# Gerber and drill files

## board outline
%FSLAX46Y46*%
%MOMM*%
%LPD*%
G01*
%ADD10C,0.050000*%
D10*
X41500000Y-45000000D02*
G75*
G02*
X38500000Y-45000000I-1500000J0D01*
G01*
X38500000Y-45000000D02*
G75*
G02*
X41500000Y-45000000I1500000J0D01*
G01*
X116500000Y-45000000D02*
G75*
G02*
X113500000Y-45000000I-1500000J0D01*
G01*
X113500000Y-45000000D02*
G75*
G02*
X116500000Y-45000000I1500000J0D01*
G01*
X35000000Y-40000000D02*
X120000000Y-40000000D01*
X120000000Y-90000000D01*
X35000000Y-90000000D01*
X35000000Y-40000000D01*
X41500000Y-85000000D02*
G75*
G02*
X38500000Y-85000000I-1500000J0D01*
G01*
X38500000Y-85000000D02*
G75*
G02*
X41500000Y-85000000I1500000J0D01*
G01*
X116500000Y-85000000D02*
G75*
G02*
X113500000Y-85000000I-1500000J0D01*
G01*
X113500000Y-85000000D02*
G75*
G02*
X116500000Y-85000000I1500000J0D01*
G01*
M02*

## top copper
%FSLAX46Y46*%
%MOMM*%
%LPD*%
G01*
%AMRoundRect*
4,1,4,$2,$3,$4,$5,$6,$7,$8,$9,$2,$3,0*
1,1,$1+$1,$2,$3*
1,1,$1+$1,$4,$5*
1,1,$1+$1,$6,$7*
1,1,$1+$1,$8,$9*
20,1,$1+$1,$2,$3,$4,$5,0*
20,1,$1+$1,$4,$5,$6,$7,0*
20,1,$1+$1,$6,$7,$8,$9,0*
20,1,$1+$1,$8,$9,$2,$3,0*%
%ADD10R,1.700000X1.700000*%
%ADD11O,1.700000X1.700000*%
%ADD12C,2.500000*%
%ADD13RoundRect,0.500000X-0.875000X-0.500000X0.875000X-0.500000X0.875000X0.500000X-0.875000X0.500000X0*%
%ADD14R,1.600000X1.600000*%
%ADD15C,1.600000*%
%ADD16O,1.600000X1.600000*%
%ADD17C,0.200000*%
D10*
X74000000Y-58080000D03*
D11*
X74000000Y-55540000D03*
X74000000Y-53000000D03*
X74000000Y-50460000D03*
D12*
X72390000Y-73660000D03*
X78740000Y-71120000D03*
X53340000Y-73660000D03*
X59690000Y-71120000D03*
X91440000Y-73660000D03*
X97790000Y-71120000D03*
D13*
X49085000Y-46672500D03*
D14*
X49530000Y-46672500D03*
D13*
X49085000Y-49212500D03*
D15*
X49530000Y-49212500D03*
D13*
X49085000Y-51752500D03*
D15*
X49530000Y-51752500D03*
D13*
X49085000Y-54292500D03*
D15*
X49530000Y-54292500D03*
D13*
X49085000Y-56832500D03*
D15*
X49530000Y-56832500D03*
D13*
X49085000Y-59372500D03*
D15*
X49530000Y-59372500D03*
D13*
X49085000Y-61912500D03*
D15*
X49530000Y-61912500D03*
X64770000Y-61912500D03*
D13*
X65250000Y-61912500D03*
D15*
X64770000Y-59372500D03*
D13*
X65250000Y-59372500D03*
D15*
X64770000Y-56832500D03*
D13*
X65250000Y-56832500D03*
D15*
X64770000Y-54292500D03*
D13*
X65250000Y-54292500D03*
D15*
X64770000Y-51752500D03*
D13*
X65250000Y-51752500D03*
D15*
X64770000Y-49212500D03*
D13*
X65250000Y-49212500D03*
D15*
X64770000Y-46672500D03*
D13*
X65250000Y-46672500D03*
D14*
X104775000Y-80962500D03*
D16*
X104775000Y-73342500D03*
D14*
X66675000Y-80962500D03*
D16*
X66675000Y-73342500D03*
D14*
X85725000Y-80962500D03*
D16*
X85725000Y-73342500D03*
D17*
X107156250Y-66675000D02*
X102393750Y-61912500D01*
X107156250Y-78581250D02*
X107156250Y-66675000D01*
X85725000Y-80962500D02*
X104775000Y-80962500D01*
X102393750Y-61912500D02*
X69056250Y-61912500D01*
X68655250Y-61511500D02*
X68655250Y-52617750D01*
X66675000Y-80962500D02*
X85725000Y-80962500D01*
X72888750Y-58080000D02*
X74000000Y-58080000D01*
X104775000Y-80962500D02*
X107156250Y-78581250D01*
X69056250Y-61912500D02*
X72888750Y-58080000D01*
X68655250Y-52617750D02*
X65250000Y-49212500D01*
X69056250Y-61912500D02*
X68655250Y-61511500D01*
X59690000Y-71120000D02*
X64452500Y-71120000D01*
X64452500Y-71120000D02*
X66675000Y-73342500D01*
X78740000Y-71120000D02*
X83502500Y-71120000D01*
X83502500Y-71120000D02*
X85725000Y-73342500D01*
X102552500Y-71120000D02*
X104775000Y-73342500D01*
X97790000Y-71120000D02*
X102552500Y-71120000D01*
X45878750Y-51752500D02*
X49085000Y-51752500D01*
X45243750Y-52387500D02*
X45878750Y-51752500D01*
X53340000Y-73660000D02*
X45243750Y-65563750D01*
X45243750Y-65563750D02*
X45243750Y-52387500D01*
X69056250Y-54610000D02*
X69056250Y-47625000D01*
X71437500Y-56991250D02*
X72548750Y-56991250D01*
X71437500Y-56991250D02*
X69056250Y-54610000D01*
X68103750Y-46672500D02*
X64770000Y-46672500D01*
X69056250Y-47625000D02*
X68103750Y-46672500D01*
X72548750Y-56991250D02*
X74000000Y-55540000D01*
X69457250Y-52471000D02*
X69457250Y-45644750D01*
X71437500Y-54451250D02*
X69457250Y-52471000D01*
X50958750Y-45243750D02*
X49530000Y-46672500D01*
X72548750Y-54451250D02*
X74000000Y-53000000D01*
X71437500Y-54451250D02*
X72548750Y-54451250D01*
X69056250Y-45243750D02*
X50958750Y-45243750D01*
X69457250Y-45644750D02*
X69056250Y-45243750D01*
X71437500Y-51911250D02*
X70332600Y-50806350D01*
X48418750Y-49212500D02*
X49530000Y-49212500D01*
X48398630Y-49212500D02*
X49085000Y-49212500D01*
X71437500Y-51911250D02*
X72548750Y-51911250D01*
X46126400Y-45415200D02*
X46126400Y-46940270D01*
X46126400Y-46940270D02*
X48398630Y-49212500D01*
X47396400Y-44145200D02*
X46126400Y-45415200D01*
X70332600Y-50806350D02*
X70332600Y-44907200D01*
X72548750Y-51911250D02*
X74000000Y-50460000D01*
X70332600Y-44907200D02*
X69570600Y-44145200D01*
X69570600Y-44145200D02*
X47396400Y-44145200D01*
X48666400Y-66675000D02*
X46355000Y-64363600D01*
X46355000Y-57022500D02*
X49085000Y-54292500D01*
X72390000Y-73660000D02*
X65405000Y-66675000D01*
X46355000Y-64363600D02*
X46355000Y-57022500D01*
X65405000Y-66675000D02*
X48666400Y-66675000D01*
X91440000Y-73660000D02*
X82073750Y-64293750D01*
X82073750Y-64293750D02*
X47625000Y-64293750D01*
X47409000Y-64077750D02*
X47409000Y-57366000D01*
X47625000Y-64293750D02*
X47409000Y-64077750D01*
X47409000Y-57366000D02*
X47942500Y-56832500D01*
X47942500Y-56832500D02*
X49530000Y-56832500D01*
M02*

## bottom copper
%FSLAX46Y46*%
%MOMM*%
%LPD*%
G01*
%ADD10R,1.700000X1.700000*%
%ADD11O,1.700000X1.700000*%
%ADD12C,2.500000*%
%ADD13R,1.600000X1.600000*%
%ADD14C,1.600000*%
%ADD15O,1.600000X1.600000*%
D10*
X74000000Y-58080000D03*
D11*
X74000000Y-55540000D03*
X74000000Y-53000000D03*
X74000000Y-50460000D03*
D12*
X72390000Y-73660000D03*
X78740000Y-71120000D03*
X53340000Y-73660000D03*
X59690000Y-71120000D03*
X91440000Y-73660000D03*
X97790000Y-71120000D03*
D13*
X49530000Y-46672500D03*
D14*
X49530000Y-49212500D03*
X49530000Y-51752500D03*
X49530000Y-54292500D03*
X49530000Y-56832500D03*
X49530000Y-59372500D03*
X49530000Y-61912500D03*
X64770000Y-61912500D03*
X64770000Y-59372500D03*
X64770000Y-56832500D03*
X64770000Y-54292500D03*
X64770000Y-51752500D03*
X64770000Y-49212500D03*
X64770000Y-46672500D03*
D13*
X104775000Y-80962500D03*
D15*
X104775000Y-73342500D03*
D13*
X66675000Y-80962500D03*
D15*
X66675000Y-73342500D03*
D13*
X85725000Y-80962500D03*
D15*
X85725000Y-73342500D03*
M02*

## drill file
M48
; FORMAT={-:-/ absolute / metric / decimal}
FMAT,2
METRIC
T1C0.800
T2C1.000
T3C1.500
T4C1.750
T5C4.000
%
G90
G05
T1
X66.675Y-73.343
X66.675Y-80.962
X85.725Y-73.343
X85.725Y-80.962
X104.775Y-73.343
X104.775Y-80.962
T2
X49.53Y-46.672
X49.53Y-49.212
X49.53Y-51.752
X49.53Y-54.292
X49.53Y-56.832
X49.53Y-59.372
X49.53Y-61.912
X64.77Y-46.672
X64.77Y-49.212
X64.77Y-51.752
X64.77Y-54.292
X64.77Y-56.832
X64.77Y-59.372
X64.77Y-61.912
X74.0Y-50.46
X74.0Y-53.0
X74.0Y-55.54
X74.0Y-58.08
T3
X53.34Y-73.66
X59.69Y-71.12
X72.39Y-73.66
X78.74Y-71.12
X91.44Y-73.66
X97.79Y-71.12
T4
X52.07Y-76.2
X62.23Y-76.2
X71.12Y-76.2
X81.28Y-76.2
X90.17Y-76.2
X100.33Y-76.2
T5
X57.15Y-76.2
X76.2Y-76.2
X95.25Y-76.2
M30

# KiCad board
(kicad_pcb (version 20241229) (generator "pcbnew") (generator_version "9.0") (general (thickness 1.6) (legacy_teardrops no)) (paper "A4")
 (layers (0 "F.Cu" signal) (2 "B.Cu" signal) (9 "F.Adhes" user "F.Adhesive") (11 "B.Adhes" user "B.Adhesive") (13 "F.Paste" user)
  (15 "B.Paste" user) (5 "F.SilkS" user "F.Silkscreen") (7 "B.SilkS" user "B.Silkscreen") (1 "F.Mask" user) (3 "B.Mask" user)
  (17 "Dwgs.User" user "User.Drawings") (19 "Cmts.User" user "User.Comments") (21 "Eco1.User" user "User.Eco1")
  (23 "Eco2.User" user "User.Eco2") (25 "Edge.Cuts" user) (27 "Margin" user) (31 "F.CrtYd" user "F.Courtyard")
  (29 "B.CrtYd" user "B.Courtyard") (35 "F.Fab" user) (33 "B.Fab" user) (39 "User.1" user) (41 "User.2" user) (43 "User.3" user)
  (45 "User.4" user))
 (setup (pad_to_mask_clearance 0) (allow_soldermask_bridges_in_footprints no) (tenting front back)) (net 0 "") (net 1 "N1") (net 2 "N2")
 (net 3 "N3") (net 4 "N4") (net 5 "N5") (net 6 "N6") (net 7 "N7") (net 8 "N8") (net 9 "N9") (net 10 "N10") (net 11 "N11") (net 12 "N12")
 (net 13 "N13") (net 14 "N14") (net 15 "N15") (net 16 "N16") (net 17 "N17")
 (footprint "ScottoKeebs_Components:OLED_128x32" (layer "F.Cu") (at 72.4 48.28)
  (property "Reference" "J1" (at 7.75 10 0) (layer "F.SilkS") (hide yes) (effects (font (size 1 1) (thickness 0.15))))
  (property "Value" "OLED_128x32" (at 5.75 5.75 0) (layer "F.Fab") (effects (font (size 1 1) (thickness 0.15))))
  (pad "1" thru_hole rect (at 1.6 9.8 180) (size 1.7 1.7) (drill 1) (layers "*.Cu" "*.Mask") (remove_unused_layers no) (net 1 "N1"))
  (pad "2" thru_hole oval (at 1.6 7.26 180) (size 1.7 1.7) (drill 1) (layers "*.Cu" "*.Mask") (remove_unused_layers no) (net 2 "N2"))
  (pad "3" thru_hole oval (at 1.6 4.72 180) (size 1.7 1.7) (drill 1) (layers "*.Cu" "*.Mask") (remove_unused_layers no) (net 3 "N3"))
  (pad "4" thru_hole oval (at 1.6 2.18 180) (size 1.7 1.7) (drill 1) (layers "*.Cu" "*.Mask") (remove_unused_layers no) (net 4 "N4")))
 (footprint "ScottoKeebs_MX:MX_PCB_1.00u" (layer "F.Cu") (at 76.2 76.2)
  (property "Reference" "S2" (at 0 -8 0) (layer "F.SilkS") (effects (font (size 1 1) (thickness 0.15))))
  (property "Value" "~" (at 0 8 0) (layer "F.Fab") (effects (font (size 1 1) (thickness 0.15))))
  (pad "" np_thru_hole circle (at -5.08 0) (size 1.75 1.75) (drill 1.75) (layers "*.Cu" "*.Mask"))
  (pad "" np_thru_hole circle (at 0 0) (size 4 4) (drill 4) (layers "*.Cu" "*.Mask"))
  (pad "" np_thru_hole circle (at 5.08 0) (size 1.75 1.75) (drill 1.75) (layers "*.Cu" "*.Mask"))
  (pad "1" thru_hole circle (at -3.81 -2.54) (size 2.5 2.5) (drill 1.5) (layers "*.Cu" "*.Mask") (remove_unused_layers no) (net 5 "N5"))
  (pad "2" thru_hole circle (at 2.54 -5.08) (size 2.5 2.5) (drill 1.5) (layers "*.Cu" "*.Mask") (remove_unused_layers no) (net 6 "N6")))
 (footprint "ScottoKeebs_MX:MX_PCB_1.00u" (layer "F.Cu") (at 57.15 76.2)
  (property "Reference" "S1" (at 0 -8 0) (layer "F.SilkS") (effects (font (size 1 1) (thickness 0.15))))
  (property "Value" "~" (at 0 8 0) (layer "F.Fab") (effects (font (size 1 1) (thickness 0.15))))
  (pad "" np_thru_hole circle (at -5.08 0) (size 1.75 1.75) (drill 1.75) (layers "*.Cu" "*.Mask"))
  (pad "" np_thru_hole circle (at 0 0) (size 4 4) (drill 4) (layers "*.Cu" "*.Mask"))
  (pad "" np_thru_hole circle (at 5.08 0) (size 1.75 1.75) (drill 1.75) (layers "*.Cu" "*.Mask"))
  (pad "1" thru_hole circle (at -3.81 -2.54) (size 2.5 2.5) (drill 1.5) (layers "*.Cu" "*.Mask") (remove_unused_layers no) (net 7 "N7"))
  (pad "2" thru_hole circle (at 2.54 -5.08) (size 2.5 2.5) (drill 1.5) (layers "*.Cu" "*.Mask") (remove_unused_layers no) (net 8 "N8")))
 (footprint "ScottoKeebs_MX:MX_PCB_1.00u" (layer "F.Cu") (at 95.25 76.2)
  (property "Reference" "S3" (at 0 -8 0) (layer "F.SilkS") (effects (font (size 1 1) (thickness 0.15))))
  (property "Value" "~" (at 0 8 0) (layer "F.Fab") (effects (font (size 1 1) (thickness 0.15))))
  (pad "" np_thru_hole circle (at -5.08 0) (size 1.75 1.75) (drill 1.75) (layers "*.Cu" "*.Mask"))
  (pad "" np_thru_hole circle (at 0 0) (size 4 4) (drill 4) (layers "*.Cu" "*.Mask"))
  (pad "" np_thru_hole circle (at 5.08 0) (size 1.75 1.75) (drill 1.75) (layers "*.Cu" "*.Mask"))
  (pad "1" thru_hole circle (at -3.81 -2.54) (size 2.5 2.5) (drill 1.5) (layers "*.Cu" "*.Mask") (remove_unused_layers no) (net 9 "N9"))
  (pad "2" thru_hole circle (at 2.54 -5.08) (size 2.5 2.5) (drill 1.5) (layers "*.Cu" "*.Mask") (remove_unused_layers no) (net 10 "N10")))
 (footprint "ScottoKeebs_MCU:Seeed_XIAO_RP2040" (layer "F.Cu") (at 57.15 54.2925)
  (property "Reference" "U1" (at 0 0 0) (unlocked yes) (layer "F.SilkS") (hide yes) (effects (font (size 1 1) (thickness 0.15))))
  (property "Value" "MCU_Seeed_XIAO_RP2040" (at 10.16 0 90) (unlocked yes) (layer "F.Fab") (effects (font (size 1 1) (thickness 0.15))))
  (pad "1" smd roundrect (at -8.065 -7.62) (size 2.75 2) (layers "F.Cu" "F.Mask" "F.Paste") (roundrect_rratio 0.25) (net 3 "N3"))
  (pad "1" thru_hole rect (at -7.62 -7.62 90) (size 1.6 1.6) (drill 1) (layers "*.Cu" "*.Mask") (remove_unused_layers no) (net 3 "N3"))
  (pad "2" smd roundrect (at -8.065 -5.08) (size 2.75 2) (layers "F.Cu" "F.Mask" "F.Paste") (roundrect_rratio 0.25) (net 4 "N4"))
  (pad "2" thru_hole circle (at -7.62 -5.08 90) (size 1.6 1.6) (drill 1) (layers "*.Cu" "*.Mask") (remove_unused_layers no) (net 4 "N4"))
  (pad "3" smd roundrect (at -8.065 -2.54) (size 2.75 2) (layers "F.Cu" "F.Mask" "F.Paste") (roundrect_rratio 0.25) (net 7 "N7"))
  (pad "3" thru_hole circle (at -7.62 -2.54 90) (size 1.6 1.6) (drill 1) (layers "*.Cu" "*.Mask") (remove_unused_layers no) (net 7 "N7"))
  (pad "4" smd roundrect (at -8.065 0) (size 2.75 2) (layers "F.Cu" "F.Mask" "F.Paste") (roundrect_rratio 0.25) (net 5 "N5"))
  (pad "4" thru_hole circle (at -7.62 0 90) (size 1.6 1.6) (drill 1) (layers "*.Cu" "*.Mask") (remove_unused_layers no) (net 5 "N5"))
  (pad "5" smd roundrect (at -8.065 2.54) (size 2.75 2) (layers "F.Cu" "F.Mask" "F.Paste") (roundrect_rratio 0.25) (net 9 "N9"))
  (pad "5" thru_hole circle (at -7.62 2.54 90) (size 1.6 1.6) (drill 1) (layers "*.Cu" "*.Mask") (remove_unused_layers no) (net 9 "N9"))
  (pad "6" smd roundrect (at -8.065 5.08) (size 2.75 2) (layers "F.Cu" "F.Mask" "F.Paste") (roundrect_rratio 0.25) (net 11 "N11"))
  (pad "6" thru_hole circle (at -7.62 5.08 90) (size 1.6 1.6) (drill 1) (layers "*.Cu" "*.Mask") (remove_unused_layers no) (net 11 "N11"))
  (pad "7" smd roundrect (at -8.065 7.62) (size 2.75 2) (layers "F.Cu" "F.Mask" "F.Paste") (roundrect_rratio 0.25) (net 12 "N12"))
  (pad "7" thru_hole circle (at -7.62 7.62 90) (size 1.6 1.6) (drill 1) (layers "*.Cu" "*.Mask") (remove_unused_layers no) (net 12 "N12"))
  (pad "8" thru_hole circle (at 7.62 7.62 90) (size 1.6 1.6) (drill 1) (layers "*.Cu" "*.Mask") (remove_unused_layers no) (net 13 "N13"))
  (pad "8" smd roundrect (at 8.1 7.62) (size 2.75 2) (layers "F.Cu" "F.Mask" "F.Paste") (roundrect_rratio 0.25) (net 13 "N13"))
  (pad "9" thru_hole circle (at 7.62 5.08 90) (size 1.6 1.6) (drill 1) (layers "*.Cu" "*.Mask") (remove_unused_layers no) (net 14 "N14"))
  (pad "9" smd roundrect (at 8.1 5.08) (size 2.75 2) (layers "F.Cu" "F.Mask" "F.Paste") (roundrect_rratio 0.25) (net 14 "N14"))
  (pad "10" thru_hole circle (at 7.62 2.54 90) (size 1.6 1.6) (drill 1) (layers "*.Cu" "*.Mask") (remove_unused_layers no) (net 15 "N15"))
  (pad "10" smd roundrect (at 8.1 2.54) (size 2.75 2) (layers "F.Cu" "F.Mask" "F.Paste") (roundrect_rratio 0.25) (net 15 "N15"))
  (pad "11" thru_hole circle (at 7.62 0 90) (size 1.6 1.6) (drill 1) (layers "*.Cu" "*.Mask") (remove_unused_layers no) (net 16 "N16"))
  (pad "11" smd roundrect (at 8.1 0) (size 2.75 2) (layers "F.Cu" "F.Mask" "F.Paste") (roundrect_rratio 0.25) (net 16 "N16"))
  (pad "12" thru_hole circle (at 7.62 -2.54 90) (size 1.6 1.6) (drill 1) (layers "*.Cu" "*.Mask") (remove_unused_layers no) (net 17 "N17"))
  (pad "12" smd roundrect (at 8.1 -2.54) (size 2.75 2) (layers "F.Cu" "F.Mask" "F.Paste") (roundrect_rratio 0.25) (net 17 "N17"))
  (pad "13" thru_hole circle (at 7.62 -5.08 90) (size 1.6 1.6) (drill 1) (layers "*.Cu" "*.Mask") (remove_unused_layers no) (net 1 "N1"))
  (pad "13" smd roundrect (at 8.1 -5.08) (size 2.75 2) (layers "F.Cu" "F.Mask" "F.Paste") (roundrect_rratio 0.25) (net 1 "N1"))
  (pad "14" thru_hole circle (at 7.62 -7.62 90) (size 1.6 1.6) (drill 1) (layers "*.Cu" "*.Mask") (remove_unused_layers no) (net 2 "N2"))
  (pad "14" smd roundrect (at 8.1 -7.62) (size 2.75 2) (layers "F.Cu" "F.Mask" "F.Paste") (roundrect_rratio 0.25) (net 2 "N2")))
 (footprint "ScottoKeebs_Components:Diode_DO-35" (layer "B.Cu") (at 104.775 80.9625 90)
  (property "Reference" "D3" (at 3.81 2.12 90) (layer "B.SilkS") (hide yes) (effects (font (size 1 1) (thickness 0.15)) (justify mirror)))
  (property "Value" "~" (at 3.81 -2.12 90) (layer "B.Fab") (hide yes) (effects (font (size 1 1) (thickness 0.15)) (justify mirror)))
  (pad "1" thru_hole rect (at 0 0 90) (size 1.6 1.6) (drill 0.8) (layers "*.Cu" "*.Mask") (remove_unused_layers no) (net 1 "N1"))
  (pad "2" thru_hole oval (at 7.62 0 90) (size 1.6 1.6) (drill 0.8) (layers "*.Cu" "*.Mask") (remove_unused_layers no) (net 10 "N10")))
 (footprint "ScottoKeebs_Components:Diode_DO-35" (layer "B.Cu") (at 66.675 80.9625 90)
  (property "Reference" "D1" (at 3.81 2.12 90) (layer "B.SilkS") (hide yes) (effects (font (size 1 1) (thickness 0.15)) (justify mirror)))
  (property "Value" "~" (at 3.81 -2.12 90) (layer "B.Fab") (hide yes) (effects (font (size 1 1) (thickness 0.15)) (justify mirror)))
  (pad "1" thru_hole rect (at 0 0 90) (size 1.6 1.6) (drill 0.8) (layers "*.Cu" "*.Mask") (remove_unused_layers no) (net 1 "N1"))
  (pad "2" thru_hole oval (at 7.62 0 90) (size 1.6 1.6) (drill 0.8) (layers "*.Cu" "*.Mask") (remove_unused_layers no) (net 8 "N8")))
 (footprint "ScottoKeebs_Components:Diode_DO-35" (layer "B.Cu") (at 85.725 80.9625 90)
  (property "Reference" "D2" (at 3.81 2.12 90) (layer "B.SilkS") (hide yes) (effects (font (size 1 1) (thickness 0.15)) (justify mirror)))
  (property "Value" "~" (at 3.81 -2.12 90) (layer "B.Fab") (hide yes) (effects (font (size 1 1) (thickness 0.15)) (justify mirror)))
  (pad "1" thru_hole rect (at 0 0 90) (size 1.6 1.6) (drill 0.8) (layers "*.Cu" "*.Mask") (remove_unused_layers no) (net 1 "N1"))
  (pad "2" thru_hole oval (at 7.62 0 90) (size 1.6 1.6) (drill 0.8) (layers "*.Cu" "*.Mask") (remove_unused_layers no) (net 6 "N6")))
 (gr_circle (center 40 45) (end 40 46.5) (stroke (width 0.05) (type default)) (fill no) (layer "Edge.Cuts"))
 (gr_circle (center 115 45) (end 115 46.5) (stroke (width 0.05) (type default)) (fill no) (layer "Edge.Cuts"))
 (gr_rect (start 35 40) (end 120 90) (stroke (width 0.05) (type default)) (fill no) (layer "Edge.Cuts"))
 (gr_circle (center 40 85) (end 40 86.5) (stroke (width 0.05) (type default)) (fill no) (layer "Edge.Cuts"))
 (gr_circle (center 115 85) (end 115 86.5) (stroke (width 0.05) (type default)) (fill no) (layer "Edge.Cuts"))
 (segment (start 107.15625 66.675) (end 102.39375 61.9125) (width 0.2) (layer "F.Cu") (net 1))
 (segment (start 107.15625 78.58125) (end 107.15625 66.675) (width 0.2) (layer "F.Cu") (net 1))
 (segment (start 85.725 80.9625) (end 104.775 80.9625) (width 0.2) (layer "F.Cu") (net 1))
 (segment (start 102.39375 61.9125) (end 69.05625 61.9125) (width 0.2) (layer "F.Cu") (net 1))
 (segment (start 68.65525 61.5115) (end 68.65525 52.61775) (width 0.2) (layer "F.Cu") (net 1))
 (segment (start 66.675 80.9625) (end 85.725 80.9625) (width 0.2) (layer "F.Cu") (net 1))
 (segment (start 72.88875 58.08) (end 74 58.08) (width 0.2) (layer "F.Cu") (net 1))
 (segment (start 104.775 80.9625) (end 107.15625 78.58125) (width 0.2) (layer "F.Cu") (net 1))
 (segment (start 69.05625 61.9125) (end 72.88875 58.08) (width 0.2) (layer "F.Cu") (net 1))
 (segment (start 68.65525 52.61775) (end 65.25 49.2125) (width 0.2) (layer "F.Cu") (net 1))
 (segment (start 69.05625 61.9125) (end 68.65525 61.5115) (width 0.2) (layer "F.Cu") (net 1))
 (segment (start 59.69 71.12) (end 64.4525 71.12) (width 0.2) (layer "F.Cu") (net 8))
 (segment (start 64.4525 71.12) (end 66.675 73.3425) (width 0.2) (layer "F.Cu") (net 8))
 (segment (start 78.74 71.12) (end 83.5025 71.12) (width 0.2) (layer "F.Cu") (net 6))
 (segment (start 83.5025 71.12) (end 85.725 73.3425) (width 0.2) (layer "F.Cu") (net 6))
 (segment (start 102.5525 71.12) (end 104.775 73.3425) (width 0.2) (layer "F.Cu") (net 10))
 (segment (start 97.79 71.12) (end 102.5525 71.12) (width 0.2) (layer "F.Cu") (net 10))
 (segment (start 45.87875 51.7525) (end 49.085 51.7525) (width 0.2) (layer "F.Cu") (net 7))
 (segment (start 45.24375 52.3875) (end 45.87875 51.7525) (width 0.2) (layer "F.Cu") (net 7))
 (segment (start 53.34 73.66) (end 45.24375 65.56375) (width 0.2) (layer "F.Cu") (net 7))
 (segment (start 45.24375 65.56375) (end 45.24375 52.3875) (width 0.2) (layer "F.Cu") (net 7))
 (segment (start 69.05625 54.61) (end 69.05625 47.625) (width 0.2) (layer "F.Cu") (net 2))
 (segment (start 71.4375 56.99125) (end 72.54875 56.99125) (width 0.2) (layer "F.Cu") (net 2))
 (segment (start 71.4375 56.99125) (end 69.05625 54.61) (width 0.2) (layer "F.Cu") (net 2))
 (segment (start 68.10375 46.6725) (end 64.77 46.6725) (width 0.2) (layer "F.Cu") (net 2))
 (segment (start 69.05625 47.625) (end 68.10375 46.6725) (width 0.2) (layer "F.Cu") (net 2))
 (segment (start 72.54875 56.99125) (end 74 55.54) (width 0.2) (layer "F.Cu") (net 2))
 (segment (start 69.45725 52.471) (end 69.45725 45.64475) (width 0.2) (layer "F.Cu") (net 3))
 (segment (start 71.4375 54.45125) (end 69.45725 52.471) (width 0.2) (layer "F.Cu") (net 3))
 (segment (start 50.95875 45.24375) (end 49.53 46.6725) (width 0.2) (layer "F.Cu") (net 3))
 (segment (start 72.54875 54.45125) (end 74 53) (width 0.2) (layer "F.Cu") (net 3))
 (segment (start 71.4375 54.45125) (end 72.54875 54.45125) (width 0.2) (layer "F.Cu") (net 3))
 (segment (start 69.05625 45.24375) (end 50.95875 45.24375) (width 0.2) (layer "F.Cu") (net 3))
 (segment (start 69.45725 45.64475) (end 69.05625 45.24375) (width 0.2) (layer "F.Cu") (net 3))
 (segment (start 71.4375 51.91125) (end 70.3326 50.80635) (width 0.2) (layer "F.Cu") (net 4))
 (segment (start 48.41875 49.2125) (end 49.53 49.2125) (width 0.2) (layer "F.Cu") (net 4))
 (segment (start 48.39863 49.2125) (end 49.085 49.2125) (width 0.2) (layer "F.Cu") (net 4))
 (segment (start 71.4375 51.91125) (end 72.54875 51.91125) (width 0.2) (layer "F.Cu") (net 4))
 (segment (start 46.1264 45.4152) (end 46.1264 46.94027) (width 0.2) (layer "F.Cu") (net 4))
 (segment (start 46.1264 46.94027) (end 48.39863 49.2125) (width 0.2) (layer "F.Cu") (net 4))
 (segment (start 47.3964 44.1452) (end 46.1264 45.4152) (width 0.2) (layer "F.Cu") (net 4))
 (segment (start 70.3326 50.80635) (end 70.3326 44.9072) (width 0.2) (layer "F.Cu") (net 4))
 (segment (start 72.54875 51.91125) (end 74 50.46) (width 0.2) (layer "F.Cu") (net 4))
 (segment (start 70.3326 44.9072) (end 69.5706 44.1452) (width 0.2) (layer "F.Cu") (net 4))
 (segment (start 69.5706 44.1452) (end 47.3964 44.1452) (width 0.2) (layer "F.Cu") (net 4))
 (segment (start 48.6664 66.675) (end 46.355 64.3636) (width 0.2) (layer "F.Cu") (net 5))
 (segment (start 46.355 57.0225) (end 49.085 54.2925) (width 0.2) (layer "F.Cu") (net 5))
 (segment (start 72.39 73.66) (end 65.405 66.675) (width 0.2) (layer "F.Cu") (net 5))
 (segment (start 46.355 64.3636) (end 46.355 57.0225) (width 0.2) (layer "F.Cu") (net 5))
 (segment (start 65.405 66.675) (end 48.6664 66.675) (width 0.2) (layer "F.Cu") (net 5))
 (segment (start 91.44 73.66) (end 82.07375 64.29375) (width 0.2) (layer "F.Cu") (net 9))
 (segment (start 82.07375 64.29375) (end 47.625 64.29375) (width 0.2) (layer "F.Cu") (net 9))
 (segment (start 47.409 64.07775) (end 47.409 57.366) (width 0.2) (layer "F.Cu") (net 9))
 (segment (start 47.625 64.29375) (end 47.409 64.07775) (width 0.2) (layer "F.Cu") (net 9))
 (segment (start 47.409 57.366) (end 47.9425 56.8325) (width 0.2) (layer "F.Cu") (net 9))
 (segment (start 47.9425 56.8325) (end 49.53 56.8325) (width 0.2) (layer "F.Cu") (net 9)))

